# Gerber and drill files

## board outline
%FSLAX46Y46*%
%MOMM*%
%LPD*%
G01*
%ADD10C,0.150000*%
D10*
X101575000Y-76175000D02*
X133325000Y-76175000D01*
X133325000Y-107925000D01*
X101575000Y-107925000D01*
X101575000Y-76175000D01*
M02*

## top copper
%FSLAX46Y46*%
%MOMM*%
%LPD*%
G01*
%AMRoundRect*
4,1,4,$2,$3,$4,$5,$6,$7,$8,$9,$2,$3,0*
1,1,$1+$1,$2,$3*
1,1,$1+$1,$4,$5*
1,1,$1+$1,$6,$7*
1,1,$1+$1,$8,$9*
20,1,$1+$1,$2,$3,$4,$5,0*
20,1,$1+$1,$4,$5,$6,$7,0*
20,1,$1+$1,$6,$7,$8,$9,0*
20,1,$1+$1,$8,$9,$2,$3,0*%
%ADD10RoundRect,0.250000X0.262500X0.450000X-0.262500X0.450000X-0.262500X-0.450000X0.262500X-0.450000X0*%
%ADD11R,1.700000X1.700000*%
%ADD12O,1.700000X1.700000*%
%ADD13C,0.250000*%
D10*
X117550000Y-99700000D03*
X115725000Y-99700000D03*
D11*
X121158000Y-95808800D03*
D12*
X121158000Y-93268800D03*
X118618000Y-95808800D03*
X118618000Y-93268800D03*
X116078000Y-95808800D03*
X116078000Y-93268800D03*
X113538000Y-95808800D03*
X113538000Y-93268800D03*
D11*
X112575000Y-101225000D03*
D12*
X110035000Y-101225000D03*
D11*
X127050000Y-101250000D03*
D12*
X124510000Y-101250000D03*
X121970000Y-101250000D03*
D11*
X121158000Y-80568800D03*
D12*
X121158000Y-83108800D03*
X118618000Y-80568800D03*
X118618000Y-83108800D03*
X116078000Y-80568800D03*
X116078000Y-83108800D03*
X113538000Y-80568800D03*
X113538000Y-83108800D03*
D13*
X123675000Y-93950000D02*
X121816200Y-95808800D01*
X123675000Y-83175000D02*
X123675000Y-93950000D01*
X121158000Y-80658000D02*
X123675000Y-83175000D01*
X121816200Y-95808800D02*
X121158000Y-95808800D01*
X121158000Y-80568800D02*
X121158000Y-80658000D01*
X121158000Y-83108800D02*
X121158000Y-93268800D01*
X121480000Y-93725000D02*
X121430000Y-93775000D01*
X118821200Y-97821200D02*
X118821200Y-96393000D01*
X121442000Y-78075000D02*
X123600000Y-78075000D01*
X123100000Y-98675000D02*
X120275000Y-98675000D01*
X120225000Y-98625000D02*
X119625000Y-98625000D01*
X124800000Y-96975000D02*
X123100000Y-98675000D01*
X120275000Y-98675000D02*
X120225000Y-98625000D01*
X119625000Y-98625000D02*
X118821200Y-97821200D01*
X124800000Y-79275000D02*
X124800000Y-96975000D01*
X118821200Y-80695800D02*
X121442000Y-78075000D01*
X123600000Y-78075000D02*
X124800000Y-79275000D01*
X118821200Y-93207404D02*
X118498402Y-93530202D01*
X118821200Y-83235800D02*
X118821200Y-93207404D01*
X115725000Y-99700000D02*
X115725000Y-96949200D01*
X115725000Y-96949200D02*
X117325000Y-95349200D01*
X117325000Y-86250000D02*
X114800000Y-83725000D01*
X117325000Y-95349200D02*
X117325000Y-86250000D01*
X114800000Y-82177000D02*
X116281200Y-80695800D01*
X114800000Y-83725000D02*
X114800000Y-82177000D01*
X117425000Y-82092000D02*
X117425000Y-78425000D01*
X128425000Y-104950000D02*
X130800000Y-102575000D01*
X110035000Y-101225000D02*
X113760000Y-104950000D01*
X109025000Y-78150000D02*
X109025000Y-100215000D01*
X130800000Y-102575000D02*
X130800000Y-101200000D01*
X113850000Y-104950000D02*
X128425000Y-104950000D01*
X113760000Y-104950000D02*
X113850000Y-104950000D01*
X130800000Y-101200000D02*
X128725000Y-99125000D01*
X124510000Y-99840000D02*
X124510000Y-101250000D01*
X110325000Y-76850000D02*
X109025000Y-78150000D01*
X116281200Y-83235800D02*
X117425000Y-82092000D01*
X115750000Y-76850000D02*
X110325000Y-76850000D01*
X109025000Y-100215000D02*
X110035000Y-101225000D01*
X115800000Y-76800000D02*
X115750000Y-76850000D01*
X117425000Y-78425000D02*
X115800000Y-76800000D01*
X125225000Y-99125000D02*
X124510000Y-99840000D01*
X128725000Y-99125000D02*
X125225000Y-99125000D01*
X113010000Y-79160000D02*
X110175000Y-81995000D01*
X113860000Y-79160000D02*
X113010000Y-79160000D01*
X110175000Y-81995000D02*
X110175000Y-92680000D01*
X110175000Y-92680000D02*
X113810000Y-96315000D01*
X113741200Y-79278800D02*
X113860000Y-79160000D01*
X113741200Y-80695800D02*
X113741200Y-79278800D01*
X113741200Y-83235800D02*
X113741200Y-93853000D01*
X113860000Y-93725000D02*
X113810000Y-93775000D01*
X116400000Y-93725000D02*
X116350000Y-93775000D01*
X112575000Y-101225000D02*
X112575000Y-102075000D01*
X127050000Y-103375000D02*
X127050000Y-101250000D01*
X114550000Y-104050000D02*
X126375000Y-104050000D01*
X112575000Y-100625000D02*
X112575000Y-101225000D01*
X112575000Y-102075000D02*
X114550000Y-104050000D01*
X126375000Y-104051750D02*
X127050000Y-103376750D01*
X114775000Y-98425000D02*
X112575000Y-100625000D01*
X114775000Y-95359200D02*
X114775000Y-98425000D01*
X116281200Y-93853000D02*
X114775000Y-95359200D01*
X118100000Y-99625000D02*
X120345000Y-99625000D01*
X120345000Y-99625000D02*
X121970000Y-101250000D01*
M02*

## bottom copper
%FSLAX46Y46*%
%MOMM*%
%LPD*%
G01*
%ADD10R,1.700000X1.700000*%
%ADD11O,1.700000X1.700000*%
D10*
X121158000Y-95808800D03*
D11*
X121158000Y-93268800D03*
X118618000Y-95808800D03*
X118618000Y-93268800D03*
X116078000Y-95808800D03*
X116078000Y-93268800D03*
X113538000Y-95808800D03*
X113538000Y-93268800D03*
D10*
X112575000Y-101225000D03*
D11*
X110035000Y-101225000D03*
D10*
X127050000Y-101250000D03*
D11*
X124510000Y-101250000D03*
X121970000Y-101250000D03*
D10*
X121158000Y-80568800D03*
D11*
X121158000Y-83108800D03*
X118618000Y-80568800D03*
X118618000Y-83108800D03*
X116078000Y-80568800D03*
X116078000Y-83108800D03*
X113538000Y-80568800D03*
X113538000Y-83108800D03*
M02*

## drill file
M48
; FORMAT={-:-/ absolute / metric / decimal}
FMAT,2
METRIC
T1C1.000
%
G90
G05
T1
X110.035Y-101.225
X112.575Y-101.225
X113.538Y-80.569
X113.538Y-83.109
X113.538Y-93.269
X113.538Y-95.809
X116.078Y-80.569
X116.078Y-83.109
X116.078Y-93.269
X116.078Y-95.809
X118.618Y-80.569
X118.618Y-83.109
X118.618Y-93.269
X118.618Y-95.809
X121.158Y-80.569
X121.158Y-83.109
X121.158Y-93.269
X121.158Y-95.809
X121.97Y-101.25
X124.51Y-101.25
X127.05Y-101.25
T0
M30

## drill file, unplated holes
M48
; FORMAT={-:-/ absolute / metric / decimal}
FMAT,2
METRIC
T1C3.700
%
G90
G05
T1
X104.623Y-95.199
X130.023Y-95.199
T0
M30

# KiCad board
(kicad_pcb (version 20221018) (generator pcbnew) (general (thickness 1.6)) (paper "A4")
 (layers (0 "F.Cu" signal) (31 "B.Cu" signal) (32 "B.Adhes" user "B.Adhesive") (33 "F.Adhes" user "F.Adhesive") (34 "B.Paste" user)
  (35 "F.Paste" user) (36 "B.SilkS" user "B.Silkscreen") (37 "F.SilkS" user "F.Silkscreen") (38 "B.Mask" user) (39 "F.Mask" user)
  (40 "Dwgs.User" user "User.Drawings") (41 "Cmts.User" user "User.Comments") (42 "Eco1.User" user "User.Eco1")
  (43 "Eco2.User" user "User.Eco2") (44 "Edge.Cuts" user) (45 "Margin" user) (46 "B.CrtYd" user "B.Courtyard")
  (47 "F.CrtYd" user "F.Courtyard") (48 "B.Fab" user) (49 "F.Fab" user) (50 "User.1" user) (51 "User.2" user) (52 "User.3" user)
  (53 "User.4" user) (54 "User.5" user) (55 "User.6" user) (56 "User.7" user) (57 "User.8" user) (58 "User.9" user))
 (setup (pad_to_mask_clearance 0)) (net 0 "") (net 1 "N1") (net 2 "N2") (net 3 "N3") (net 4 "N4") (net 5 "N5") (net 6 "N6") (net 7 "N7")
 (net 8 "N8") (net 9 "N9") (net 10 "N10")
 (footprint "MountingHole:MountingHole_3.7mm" (layer "F.Cu") (at 104.6226 95.1992)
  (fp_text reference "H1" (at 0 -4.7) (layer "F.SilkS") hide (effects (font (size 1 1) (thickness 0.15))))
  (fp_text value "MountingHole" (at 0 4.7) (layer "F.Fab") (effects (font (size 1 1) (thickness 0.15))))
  (pad "" np_thru_hole circle (at 0 0) (size 3.7 3.7) (drill 3.7) (layers "*.Cu" "*.Mask")))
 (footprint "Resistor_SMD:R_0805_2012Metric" (layer "F.Cu") (at 116.6375 99.7 180)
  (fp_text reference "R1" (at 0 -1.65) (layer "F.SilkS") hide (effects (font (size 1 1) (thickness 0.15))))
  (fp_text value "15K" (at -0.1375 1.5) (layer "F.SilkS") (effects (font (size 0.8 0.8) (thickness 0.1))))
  (pad "1" smd roundrect (at -0.9125 0 180) (size 1.025 1.4) (layers "F.Cu" "F.Paste" "F.Mask") (roundrect_rratio 0.243902439) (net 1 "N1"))
  (pad "2" smd roundrect (at 0.9125 0 180) (size 1.025 1.4) (layers "F.Cu" "F.Paste" "F.Mask") (roundrect_rratio 0.243902439) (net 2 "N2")))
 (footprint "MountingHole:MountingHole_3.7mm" (layer "F.Cu") (at 130.0226 95.1992)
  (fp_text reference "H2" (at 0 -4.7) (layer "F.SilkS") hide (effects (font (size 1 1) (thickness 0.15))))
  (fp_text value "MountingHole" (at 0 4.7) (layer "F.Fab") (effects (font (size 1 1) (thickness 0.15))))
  (pad "" np_thru_hole circle (at 0 0) (size 3.7 3.7) (drill 3.7) (layers "*.Cu" "*.Mask")))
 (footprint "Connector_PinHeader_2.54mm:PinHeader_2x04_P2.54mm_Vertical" (layer "B.Cu") (at 121.158 95.8088 90)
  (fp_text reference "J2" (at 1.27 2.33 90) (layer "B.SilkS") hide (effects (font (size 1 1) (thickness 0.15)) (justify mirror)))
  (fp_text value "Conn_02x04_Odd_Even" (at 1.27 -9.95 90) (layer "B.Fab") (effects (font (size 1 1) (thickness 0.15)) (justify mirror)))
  (pad "1" thru_hole rect (at 0 0 90) (size 1.7 1.7) (drill 1) (layers "*.Cu" "*.Mask") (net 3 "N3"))
  (pad "2" thru_hole oval (at 2.54 0 90) (size 1.7 1.7) (drill 1) (layers "*.Cu" "*.Mask") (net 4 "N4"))
  (pad "3" thru_hole oval (at 0 -2.54 90) (size 1.7 1.7) (drill 1) (layers "*.Cu" "*.Mask") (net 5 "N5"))
  (pad "4" thru_hole oval (at 2.54 -2.54 90) (size 1.7 1.7) (drill 1) (layers "*.Cu" "*.Mask") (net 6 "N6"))
  (pad "5" thru_hole oval (at 0 -5.08 90) (size 1.7 1.7) (drill 1) (layers "*.Cu" "*.Mask") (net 2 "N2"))
  (pad "6" thru_hole oval (at 2.54 -5.08 90) (size 1.7 1.7) (drill 1) (layers "*.Cu" "*.Mask") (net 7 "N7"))
  (pad "7" thru_hole oval (at 0 -7.62 90) (size 1.7 1.7) (drill 1) (layers "*.Cu" "*.Mask") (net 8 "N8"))
  (pad "8" thru_hole oval (at 2.54 -7.62 90) (size 1.7 1.7) (drill 1) (layers "*.Cu" "*.Mask") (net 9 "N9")))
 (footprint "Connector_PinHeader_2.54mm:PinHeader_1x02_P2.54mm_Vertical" (layer "B.Cu") (at 112.575 101.225 90)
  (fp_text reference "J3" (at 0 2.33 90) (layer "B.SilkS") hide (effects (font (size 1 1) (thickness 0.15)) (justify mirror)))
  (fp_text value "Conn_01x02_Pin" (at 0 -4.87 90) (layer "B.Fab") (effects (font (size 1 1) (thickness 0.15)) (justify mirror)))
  (pad "1" thru_hole rect (at 0 0 90) (size 1.7 1.7) (drill 1) (layers "*.Cu" "*.Mask") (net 7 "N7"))
  (pad "2" thru_hole oval (at 0 -2.54 90) (size 1.7 1.7) (drill 1) (layers "*.Cu" "*.Mask") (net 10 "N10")))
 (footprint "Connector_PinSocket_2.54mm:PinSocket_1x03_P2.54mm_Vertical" (layer "B.Cu") (at 127.05 101.25 90)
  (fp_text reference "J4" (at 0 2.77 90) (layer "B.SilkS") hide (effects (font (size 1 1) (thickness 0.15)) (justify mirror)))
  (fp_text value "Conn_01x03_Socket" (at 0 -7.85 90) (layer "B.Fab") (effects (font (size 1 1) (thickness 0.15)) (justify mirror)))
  (pad "1" thru_hole rect (at 0 0 90) (size 1.7 1.7) (drill 1) (layers "*.Cu" "*.Mask") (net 7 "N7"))
  (pad "2" thru_hole oval (at 0 -2.54 90) (size 1.7 1.7) (drill 1) (layers "*.Cu" "*.Mask") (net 10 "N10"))
  (pad "3" thru_hole oval (at 0 -5.08 90) (size 1.7 1.7) (drill 1) (layers "*.Cu" "*.Mask") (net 1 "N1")))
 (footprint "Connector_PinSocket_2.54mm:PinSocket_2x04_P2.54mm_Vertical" (layer "B.Cu") (at 121.158 80.5688 90)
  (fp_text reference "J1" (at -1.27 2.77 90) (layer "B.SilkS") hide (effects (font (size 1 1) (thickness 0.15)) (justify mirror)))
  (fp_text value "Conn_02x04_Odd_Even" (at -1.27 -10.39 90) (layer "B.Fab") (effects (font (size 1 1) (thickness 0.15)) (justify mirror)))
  (pad "1" thru_hole rect (at 0 0 90) (size 1.7 1.7) (drill 1) (layers "*.Cu" "*.Mask") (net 3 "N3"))
  (pad "2" thru_hole oval (at -2.54 0 90) (size 1.7 1.7) (drill 1) (layers "*.Cu" "*.Mask") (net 4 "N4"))
  (pad "3" thru_hole oval (at 0 -2.54 90) (size 1.7 1.7) (drill 1) (layers "*.Cu" "*.Mask") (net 5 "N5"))
  (pad "4" thru_hole oval (at -2.54 -2.54 90) (size 1.7 1.7) (drill 1) (layers "*.Cu" "*.Mask") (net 6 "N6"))
  (pad "5" thru_hole oval (at 0 -5.08 90) (size 1.7 1.7) (drill 1) (layers "*.Cu" "*.Mask") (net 2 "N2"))
  (pad "6" thru_hole oval (at -2.54 -5.08 90) (size 1.7 1.7) (drill 1) (layers "*.Cu" "*.Mask") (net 10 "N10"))
  (pad "7" thru_hole oval (at 0 -7.62 90) (size 1.7 1.7) (drill 1) (layers "*.Cu" "*.Mask") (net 8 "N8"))
  (pad "8" thru_hole oval (at -2.54 -7.62 90) (size 1.7 1.7) (drill 1) (layers "*.Cu" "*.Mask") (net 9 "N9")))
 (gr_rect (start 101.575 76.175) (end 133.325 107.925) (stroke (width 0.15) (type default)) (fill none) (layer "Edge.Cuts"))
 (segment (start 121.8162 95.8088) (end 121.158 95.8088) (width 0.25) (layer "F.Cu") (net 3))
 (segment (start 121.158 80.5688) (end 121.158 80.658) (width 0.25) (layer "F.Cu") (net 3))
 (segment (start 121.158 80.658) (end 123.675 83.175) (width 0.25) (layer "F.Cu") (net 3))
 (segment (start 123.675 83.175) (end 123.675 93.95) (width 0.25) (layer "F.Cu") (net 3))
 (segment (start 123.675 93.95) (end 121.8162 95.8088) (width 0.25) (layer "F.Cu") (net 3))
 (segment (start 121.158 83.1088) (end 121.158 93.2688) (width 0.25) (layer "F.Cu") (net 4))
 (segment (start 121.48 93.725) (end 121.43 93.775) (width 0.25) (layer "F.Cu") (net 4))
 (segment (start 118.8212 97.8212) (end 118.8212 96.393) (width 0.25) (layer "F.Cu") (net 5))
 (segment (start 121.442 78.075) (end 123.6 78.075) (width 0.25) (layer "F.Cu") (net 5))
 (segment (start 123.1 98.675) (end 120.275 98.675) (width 0.25) (layer "F.Cu") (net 5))
 (segment (start 120.225 98.625) (end 119.625 98.625) (width 0.25) (layer "F.Cu") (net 5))
 (segment (start 124.8 96.975) (end 123.1 98.675) (width 0.25) (layer "F.Cu") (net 5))
 (segment (start 120.275 98.675) (end 120.225 98.625) (width 0.25) (layer "F.Cu") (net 5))
 (segment (start 119.625 98.625) (end 118.8212 97.8212) (width 0.25) (layer "F.Cu") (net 5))
 (segment (start 124.8 79.275) (end 124.8 96.975) (width 0.25) (layer "F.Cu") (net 5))
 (segment (start 118.8212 80.6958) (end 121.442 78.075) (width 0.25) (layer "F.Cu") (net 5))
 (segment (start 123.6 78.075) (end 124.8 79.275) (width 0.25) (layer "F.Cu") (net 5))
 (segment (start 118.8212 93.207404) (end 118.498402 93.530202) (width 0.25) (layer "F.Cu") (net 6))
 (segment (start 118.8212 83.2358) (end 118.8212 93.207404) (width 0.25) (layer "F.Cu") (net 6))
 (segment (start 115.725 99.7) (end 115.725 96.9492) (width 0.25) (layer "F.Cu") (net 2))
 (segment (start 115.725 96.9492) (end 117.325 95.3492) (width 0.25) (layer "F.Cu") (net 2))
 (segment (start 117.325 86.25) (end 114.8 83.725) (width 0.25) (layer "F.Cu") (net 2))
 (segment (start 117.325 95.3492) (end 117.325 86.25) (width 0.25) (layer "F.Cu") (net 2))
 (segment (start 114.8 82.177) (end 116.2812 80.6958) (width 0.25) (layer "F.Cu") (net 2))
 (segment (start 114.8 83.725) (end 114.8 82.177) (width 0.25) (layer "F.Cu") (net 2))
 (segment (start 117.425 82.092) (end 117.425 78.425) (width 0.25) (layer "F.Cu") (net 10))
 (segment (start 128.425 104.95) (end 130.8 102.575) (width 0.25) (layer "F.Cu") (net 10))
 (segment (start 110.035 101.225) (end 113.76 104.95) (width 0.25) (layer "F.Cu") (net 10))
 (segment (start 109.025 78.15) (end 109.025 100.215) (width 0.25) (layer "F.Cu") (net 10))
 (segment (start 130.8 102.575) (end 130.8 101.2) (width 0.25) (layer "F.Cu") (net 10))
 (segment (start 113.85 104.95) (end 128.425 104.95) (width 0.25) (layer "F.Cu") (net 10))
 (segment (start 113.76 104.95) (end 113.85 104.95) (width 0.25) (layer "F.Cu") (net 10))
 (segment (start 130.8 101.2) (end 128.725 99.125) (width 0.25) (layer "F.Cu") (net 10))
 (segment (start 124.51 99.84) (end 124.51 101.25) (width 0.25) (layer "F.Cu") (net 10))
 (segment (start 110.325 76.85) (end 109.025 78.15) (width 0.25) (layer "F.Cu") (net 10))
 (segment (start 116.2812 83.2358) (end 117.425 82.092) (width 0.25) (layer "F.Cu") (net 10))
 (segment (start 115.75 76.85) (end 110.325 76.85) (width 0.25) (layer "F.Cu") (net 10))
 (segment (start 109.025 100.215) (end 110.035 101.225) (width 0.25) (layer "F.Cu") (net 10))
 (segment (start 115.8 76.8) (end 115.75 76.85) (width 0.25) (layer "F.Cu") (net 10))
 (segment (start 117.425 78.425) (end 115.8 76.8) (width 0.25) (layer "F.Cu") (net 10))
 (segment (start 125.225 99.125) (end 124.51 99.84) (width 0.25) (layer "F.Cu") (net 10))
 (segment (start 128.725 99.125) (end 125.225 99.125) (width 0.25) (layer "F.Cu") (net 10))
 (segment (start 113.01 79.16) (end 110.175 81.995) (width 0.25) (layer "F.Cu") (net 8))
 (segment (start 113.86 79.16) (end 113.01 79.16) (width 0.25) (layer "F.Cu") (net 8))
 (segment (start 110.175 81.995) (end 110.175 92.68) (width 0.25) (layer "F.Cu") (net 8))
 (segment (start 110.175 92.68) (end 113.81 96.315) (width 0.25) (layer "F.Cu") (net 8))
 (segment (start 113.7412 79.2788) (end 113.86 79.16) (width 0.25) (layer "F.Cu") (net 8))
 (segment (start 113.7412 80.6958) (end 113.7412 79.2788) (width 0.25) (layer "F.Cu") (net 8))
 (segment (start 113.7412 83.2358) (end 113.7412 93.853) (width 0.25) (layer "F.Cu") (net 9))
 (segment (start 113.86 93.725) (end 113.81 93.775) (width 0.25) (layer "F.Cu") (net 9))
 (segment (start 116.4 93.725) (end 116.35 93.775) (width 0.25) (layer "F.Cu") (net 7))
 (segment (start 112.575 101.225) (end 112.575 102.075) (width 0.25) (layer "F.Cu") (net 7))
 (segment (start 127.05 103.375) (end 127.05 101.25) (width 0.25) (layer "F.Cu") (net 7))
 (segment (start 114.55 104.05) (end 126.375 104.05) (width 0.25) (layer "F.Cu") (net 7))
 (segment (start 112.575 100.625) (end 112.575 101.225) (width 0.25) (layer "F.Cu") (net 7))
 (segment (start 112.575 102.075) (end 114.55 104.05) (width 0.25) (layer "F.Cu") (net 7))
 (segment (start 126.375 104.05175) (end 127.05 103.37675) (width 0.25) (layer "F.Cu") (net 7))
 (segment (start 114.775 98.425) (end 112.575 100.625) (width 0.25) (layer "F.Cu") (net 7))
 (segment (start 114.775 95.3592) (end 114.775 98.425) (width 0.25) (layer "F.Cu") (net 7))
 (segment (start 116.2812 93.853) (end 114.775 95.3592) (width 0.25) (layer "F.Cu") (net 7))
 (segment (start 118.1 99.625) (end 120.345 99.625) (width 0.25) (layer "F.Cu") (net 1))
 (segment (start 120.345 99.625) (end 121.97 101.25) (width 0.25) (layer "F.Cu") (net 1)))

